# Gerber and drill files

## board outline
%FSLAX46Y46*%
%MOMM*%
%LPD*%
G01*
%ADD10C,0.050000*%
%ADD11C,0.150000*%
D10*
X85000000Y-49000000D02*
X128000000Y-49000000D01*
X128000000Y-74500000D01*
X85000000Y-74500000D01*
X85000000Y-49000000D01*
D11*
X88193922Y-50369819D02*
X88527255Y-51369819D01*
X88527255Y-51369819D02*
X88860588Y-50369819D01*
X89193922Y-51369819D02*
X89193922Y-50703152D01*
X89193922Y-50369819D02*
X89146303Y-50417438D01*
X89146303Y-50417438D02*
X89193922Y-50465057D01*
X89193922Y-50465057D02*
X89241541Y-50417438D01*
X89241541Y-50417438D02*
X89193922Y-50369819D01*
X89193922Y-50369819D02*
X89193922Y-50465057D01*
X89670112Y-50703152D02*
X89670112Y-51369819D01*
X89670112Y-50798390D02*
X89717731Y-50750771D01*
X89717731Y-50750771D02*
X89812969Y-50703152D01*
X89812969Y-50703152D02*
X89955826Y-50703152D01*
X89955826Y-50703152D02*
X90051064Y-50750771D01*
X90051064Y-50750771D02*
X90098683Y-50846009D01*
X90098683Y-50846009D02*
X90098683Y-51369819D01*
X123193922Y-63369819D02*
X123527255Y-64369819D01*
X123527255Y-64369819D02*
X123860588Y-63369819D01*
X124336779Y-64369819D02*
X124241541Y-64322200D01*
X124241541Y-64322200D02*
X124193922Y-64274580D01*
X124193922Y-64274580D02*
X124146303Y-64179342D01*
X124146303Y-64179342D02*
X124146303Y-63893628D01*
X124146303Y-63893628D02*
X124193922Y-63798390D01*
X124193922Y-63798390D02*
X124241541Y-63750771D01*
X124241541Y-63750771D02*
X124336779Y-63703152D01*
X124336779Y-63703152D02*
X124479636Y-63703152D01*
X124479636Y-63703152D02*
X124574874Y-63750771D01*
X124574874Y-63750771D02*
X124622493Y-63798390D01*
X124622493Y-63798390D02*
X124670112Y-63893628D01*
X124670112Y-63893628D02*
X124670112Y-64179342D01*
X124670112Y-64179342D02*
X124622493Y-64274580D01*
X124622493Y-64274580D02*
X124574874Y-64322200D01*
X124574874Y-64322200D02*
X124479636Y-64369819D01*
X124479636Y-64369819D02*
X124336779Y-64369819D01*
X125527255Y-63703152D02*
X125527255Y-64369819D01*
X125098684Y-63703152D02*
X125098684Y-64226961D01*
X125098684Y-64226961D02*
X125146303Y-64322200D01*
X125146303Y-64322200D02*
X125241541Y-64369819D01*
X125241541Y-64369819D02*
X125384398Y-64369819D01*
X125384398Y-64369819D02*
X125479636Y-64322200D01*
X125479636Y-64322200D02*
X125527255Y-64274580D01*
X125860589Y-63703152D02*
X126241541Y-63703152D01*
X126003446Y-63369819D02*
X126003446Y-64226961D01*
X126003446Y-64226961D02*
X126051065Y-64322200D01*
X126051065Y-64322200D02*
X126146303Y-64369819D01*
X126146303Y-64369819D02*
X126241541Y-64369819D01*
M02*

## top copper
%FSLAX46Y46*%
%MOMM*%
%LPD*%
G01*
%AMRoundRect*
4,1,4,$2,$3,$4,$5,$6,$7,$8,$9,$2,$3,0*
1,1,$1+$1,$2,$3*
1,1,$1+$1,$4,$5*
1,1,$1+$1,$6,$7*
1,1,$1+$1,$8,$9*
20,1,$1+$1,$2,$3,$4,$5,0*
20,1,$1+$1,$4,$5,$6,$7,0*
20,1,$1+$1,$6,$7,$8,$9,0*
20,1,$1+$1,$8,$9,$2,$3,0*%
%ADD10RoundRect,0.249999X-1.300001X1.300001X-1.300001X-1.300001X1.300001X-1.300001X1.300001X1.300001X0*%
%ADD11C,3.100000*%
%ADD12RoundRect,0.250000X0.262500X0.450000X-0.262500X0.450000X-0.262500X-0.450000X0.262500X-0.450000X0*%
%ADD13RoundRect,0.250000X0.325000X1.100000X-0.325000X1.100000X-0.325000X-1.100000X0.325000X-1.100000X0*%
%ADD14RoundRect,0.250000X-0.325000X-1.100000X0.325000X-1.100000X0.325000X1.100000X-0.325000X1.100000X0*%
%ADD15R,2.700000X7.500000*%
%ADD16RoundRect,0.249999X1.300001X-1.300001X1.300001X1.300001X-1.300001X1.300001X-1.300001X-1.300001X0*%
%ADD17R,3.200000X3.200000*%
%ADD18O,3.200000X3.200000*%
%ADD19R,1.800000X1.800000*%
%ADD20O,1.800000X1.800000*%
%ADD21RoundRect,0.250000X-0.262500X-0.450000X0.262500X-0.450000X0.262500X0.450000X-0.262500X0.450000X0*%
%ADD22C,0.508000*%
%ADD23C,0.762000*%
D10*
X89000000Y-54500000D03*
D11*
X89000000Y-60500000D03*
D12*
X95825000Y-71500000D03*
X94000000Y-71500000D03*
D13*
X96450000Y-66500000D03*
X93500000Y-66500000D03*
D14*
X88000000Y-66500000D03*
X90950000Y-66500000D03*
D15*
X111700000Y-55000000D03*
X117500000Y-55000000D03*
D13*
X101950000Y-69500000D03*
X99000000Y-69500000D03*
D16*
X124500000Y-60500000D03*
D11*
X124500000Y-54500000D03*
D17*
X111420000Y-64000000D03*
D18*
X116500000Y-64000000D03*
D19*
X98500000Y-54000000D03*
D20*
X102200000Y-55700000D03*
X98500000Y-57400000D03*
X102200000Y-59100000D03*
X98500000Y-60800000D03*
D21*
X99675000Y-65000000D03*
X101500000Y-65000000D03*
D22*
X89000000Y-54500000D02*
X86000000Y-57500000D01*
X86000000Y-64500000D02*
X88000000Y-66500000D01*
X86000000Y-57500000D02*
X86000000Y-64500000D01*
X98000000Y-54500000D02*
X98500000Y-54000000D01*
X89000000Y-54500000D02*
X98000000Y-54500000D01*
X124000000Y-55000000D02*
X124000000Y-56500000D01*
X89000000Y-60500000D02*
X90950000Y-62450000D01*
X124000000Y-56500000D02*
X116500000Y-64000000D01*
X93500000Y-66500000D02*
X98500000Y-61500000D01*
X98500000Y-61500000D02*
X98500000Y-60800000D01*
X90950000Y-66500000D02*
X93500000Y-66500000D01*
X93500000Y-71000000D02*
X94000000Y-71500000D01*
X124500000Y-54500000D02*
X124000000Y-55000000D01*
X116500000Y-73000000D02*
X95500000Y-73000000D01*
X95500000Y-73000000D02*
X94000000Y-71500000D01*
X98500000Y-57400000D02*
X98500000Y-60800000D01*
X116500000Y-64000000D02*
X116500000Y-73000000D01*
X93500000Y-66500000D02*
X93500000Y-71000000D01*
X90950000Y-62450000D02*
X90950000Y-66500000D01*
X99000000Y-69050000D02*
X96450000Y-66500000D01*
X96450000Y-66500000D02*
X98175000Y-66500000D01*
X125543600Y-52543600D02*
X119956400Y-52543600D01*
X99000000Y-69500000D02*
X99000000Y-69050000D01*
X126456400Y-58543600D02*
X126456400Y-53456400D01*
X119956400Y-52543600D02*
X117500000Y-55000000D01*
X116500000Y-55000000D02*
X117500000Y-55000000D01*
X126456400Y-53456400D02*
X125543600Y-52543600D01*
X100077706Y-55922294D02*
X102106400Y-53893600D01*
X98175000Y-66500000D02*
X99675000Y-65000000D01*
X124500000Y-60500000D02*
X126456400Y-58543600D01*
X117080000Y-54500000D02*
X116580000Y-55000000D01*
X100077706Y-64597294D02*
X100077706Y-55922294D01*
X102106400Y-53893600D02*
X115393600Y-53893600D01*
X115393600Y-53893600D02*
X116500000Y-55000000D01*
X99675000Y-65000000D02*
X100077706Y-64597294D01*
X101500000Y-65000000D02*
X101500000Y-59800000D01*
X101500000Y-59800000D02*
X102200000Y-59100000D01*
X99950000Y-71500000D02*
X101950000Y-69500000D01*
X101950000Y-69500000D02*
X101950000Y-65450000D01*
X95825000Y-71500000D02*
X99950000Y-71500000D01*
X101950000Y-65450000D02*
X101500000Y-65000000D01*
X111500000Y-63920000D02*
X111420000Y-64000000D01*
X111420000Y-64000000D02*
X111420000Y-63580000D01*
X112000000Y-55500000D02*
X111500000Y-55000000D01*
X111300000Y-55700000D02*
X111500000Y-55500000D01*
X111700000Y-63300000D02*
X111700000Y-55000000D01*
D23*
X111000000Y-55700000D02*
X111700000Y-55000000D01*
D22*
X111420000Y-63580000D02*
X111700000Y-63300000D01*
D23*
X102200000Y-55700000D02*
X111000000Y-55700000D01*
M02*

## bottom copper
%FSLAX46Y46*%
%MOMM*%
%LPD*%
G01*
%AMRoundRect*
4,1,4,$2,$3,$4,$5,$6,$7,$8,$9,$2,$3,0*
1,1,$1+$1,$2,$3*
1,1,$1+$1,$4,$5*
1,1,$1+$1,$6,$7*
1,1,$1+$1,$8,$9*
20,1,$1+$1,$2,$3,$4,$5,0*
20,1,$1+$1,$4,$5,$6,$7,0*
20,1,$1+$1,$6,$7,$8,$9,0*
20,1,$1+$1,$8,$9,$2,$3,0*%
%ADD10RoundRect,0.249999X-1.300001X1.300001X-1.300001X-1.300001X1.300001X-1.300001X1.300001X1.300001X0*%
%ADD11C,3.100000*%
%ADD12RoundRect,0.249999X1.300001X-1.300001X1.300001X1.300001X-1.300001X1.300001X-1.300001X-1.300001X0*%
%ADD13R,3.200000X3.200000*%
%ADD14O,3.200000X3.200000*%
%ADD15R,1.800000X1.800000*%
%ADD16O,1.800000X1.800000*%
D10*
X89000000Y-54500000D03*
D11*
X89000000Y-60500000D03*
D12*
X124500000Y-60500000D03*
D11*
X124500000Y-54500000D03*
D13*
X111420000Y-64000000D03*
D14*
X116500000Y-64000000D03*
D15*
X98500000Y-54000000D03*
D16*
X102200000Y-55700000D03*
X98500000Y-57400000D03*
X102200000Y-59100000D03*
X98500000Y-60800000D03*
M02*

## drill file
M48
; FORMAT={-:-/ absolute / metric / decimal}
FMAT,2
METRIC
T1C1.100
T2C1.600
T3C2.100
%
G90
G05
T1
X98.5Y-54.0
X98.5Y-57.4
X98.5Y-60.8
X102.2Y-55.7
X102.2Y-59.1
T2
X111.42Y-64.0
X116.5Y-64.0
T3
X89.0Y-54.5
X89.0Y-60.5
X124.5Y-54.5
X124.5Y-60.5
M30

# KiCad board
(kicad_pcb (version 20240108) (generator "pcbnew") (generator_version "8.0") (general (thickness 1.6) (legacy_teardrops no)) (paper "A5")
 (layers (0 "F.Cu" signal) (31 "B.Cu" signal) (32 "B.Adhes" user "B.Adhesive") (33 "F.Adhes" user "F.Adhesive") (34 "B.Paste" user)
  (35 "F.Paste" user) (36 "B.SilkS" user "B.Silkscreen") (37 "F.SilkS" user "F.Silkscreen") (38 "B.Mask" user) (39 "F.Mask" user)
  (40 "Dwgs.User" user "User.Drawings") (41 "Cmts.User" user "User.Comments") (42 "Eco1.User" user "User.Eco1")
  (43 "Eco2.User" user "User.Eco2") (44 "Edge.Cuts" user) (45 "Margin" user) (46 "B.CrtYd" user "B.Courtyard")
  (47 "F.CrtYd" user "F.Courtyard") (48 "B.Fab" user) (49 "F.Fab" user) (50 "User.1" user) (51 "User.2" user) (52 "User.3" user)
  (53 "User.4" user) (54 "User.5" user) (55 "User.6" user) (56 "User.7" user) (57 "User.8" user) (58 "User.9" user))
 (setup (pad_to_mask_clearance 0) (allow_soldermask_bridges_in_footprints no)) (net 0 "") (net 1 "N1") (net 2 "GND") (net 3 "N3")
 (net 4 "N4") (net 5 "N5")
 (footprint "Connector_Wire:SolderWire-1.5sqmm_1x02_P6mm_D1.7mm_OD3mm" (layer "F.Cu") (at 89 54.5 -90)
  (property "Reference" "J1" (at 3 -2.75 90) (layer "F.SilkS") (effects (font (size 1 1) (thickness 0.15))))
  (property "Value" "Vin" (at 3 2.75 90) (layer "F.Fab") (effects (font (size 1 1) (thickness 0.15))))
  (pad "1" thru_hole roundrect (at 0 0 270) (size 3.1 3.1) (drill 2.1) (layers "*.Cu" "*.Mask") (remove_unused_layers no)
   (roundrect_rratio 0.080645) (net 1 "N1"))
  (pad "2" thru_hole circle (at 6 0 270) (size 3.1 3.1) (drill 2.1) (layers "*.Cu" "*.Mask") (remove_unused_layers no) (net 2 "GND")))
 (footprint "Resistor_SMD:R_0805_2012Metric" (layer "F.Cu") (at 94.9125 71.5 180)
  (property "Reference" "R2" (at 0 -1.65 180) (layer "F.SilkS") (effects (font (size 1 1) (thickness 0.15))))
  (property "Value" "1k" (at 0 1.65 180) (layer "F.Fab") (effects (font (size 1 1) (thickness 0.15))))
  (pad "1" smd roundrect (at -0.9125 0 180) (size 1.025 1.4) (layers "F.Cu" "F.Paste" "F.Mask") (roundrect_rratio 0.243902) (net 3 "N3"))
  (pad "2" smd roundrect (at 0.9125 0 180) (size 1.025 1.4) (layers "F.Cu" "F.Paste" "F.Mask") (roundrect_rratio 0.243902) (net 2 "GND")))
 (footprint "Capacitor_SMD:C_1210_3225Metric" (layer "F.Cu") (at 94.975 66.5 180)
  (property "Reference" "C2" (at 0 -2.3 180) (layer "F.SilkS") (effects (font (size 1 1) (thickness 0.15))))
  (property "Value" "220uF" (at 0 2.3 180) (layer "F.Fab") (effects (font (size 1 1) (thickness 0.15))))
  (pad "1" smd roundrect (at -1.475 0 180) (size 1.15 2.7) (layers "F.Cu" "F.Paste" "F.Mask") (roundrect_rratio 0.217391) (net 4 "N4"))
  (pad "2" smd roundrect (at 1.475 0 180) (size 1.15 2.7) (layers "F.Cu" "F.Paste" "F.Mask") (roundrect_rratio 0.217391) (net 2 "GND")))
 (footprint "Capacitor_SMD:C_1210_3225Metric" (layer "F.Cu") (at 89.475 66.5)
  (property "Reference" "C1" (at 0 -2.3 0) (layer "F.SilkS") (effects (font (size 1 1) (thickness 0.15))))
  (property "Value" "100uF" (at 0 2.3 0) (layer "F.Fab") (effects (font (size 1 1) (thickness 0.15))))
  (pad "1" smd roundrect (at -1.475 0) (size 1.15 2.7) (layers "F.Cu" "F.Paste" "F.Mask") (roundrect_rratio 0.217391) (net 1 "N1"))
  (pad "2" smd roundrect (at 1.475 0) (size 1.15 2.7) (layers "F.Cu" "F.Paste" "F.Mask") (roundrect_rratio 0.217391) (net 2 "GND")))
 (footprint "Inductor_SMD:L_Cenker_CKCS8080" (layer "F.Cu") (at 114.6 55)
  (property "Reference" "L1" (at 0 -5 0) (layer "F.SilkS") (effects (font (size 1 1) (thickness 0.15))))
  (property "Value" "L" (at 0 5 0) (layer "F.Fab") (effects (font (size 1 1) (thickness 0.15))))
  (pad "1" smd rect (at -2.9 0) (size 2.7 7.5) (layers "F.Cu" "F.Paste" "F.Mask") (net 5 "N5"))
  (pad "2" smd rect (at 2.9 0) (size 2.7 7.5) (layers "F.Cu" "F.Paste" "F.Mask") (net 4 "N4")))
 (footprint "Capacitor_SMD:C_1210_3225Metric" (layer "F.Cu") (at 100.475 69.5 180)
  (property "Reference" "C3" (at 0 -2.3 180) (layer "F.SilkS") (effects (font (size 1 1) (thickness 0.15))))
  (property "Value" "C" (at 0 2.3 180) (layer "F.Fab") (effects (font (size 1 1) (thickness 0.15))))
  (pad "1" smd roundrect (at -1.475 0 180) (size 1.15 2.7) (layers "F.Cu" "F.Paste" "F.Mask") (roundrect_rratio 0.217391) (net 3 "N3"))
  (pad "2" smd roundrect (at 1.475 0 180) (size 1.15 2.7) (layers "F.Cu" "F.Paste" "F.Mask") (roundrect_rratio 0.217391) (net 4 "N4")))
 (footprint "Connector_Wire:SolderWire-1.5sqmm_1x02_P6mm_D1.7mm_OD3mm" (layer "F.Cu") (at 124.5 60.5 90)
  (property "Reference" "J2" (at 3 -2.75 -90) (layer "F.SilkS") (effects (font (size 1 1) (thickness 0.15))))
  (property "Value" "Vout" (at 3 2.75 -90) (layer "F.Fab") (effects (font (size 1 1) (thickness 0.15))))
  (pad "1" thru_hole roundrect (at 0 0 90) (size 3.1 3.1) (drill 2.1) (layers "*.Cu" "*.Mask") (remove_unused_layers no)
   (roundrect_rratio 0.080645) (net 4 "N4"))
  (pad "2" thru_hole circle (at 6 0 90) (size 3.1 3.1) (drill 2.1) (layers "*.Cu" "*.Mask") (remove_unused_layers no) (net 2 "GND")))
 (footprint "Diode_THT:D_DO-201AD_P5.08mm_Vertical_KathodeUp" (layer "F.Cu") (at 111.42 64)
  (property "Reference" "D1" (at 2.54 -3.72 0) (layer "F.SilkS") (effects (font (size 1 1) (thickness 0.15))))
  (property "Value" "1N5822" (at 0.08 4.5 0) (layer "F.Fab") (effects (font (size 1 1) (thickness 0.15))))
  (pad "1" thru_hole rect (at 0 0) (size 3.2 3.2) (drill 1.6) (layers "*.Cu" "*.Mask") (remove_unused_layers no) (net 5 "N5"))
  (pad "2" thru_hole oval (at 5.08 0) (size 3.2 3.2) (drill 1.6) (layers "*.Cu" "*.Mask") (remove_unused_layers no) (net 2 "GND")))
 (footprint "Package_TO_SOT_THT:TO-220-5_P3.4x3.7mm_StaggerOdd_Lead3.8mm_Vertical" (layer "F.Cu") (at 98.5 54 -90)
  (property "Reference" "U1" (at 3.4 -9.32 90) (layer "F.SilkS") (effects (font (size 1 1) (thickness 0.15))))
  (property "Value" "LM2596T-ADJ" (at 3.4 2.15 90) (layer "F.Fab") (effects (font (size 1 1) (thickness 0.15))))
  (pad "1" thru_hole rect (at 0 0 270) (size 1.8 1.8) (drill 1.1) (layers "*.Cu" "*.Mask") (remove_unused_layers no) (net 1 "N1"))
  (pad "2" thru_hole oval (at 1.7 -3.7 270) (size 1.8 1.8) (drill 1.1) (layers "*.Cu" "*.Mask") (remove_unused_layers no) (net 5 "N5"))
  (pad "3" thru_hole oval (at 3.4 0 270) (size 1.8 1.8) (drill 1.1) (layers "*.Cu" "*.Mask") (remove_unused_layers no) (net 2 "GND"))
  (pad "4" thru_hole oval (at 5.1 -3.7 270) (size 1.8 1.8) (drill 1.1) (layers "*.Cu" "*.Mask") (remove_unused_layers no) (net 3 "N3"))
  (pad "5" thru_hole oval (at 6.8 0 270) (size 1.8 1.8) (drill 1.1) (layers "*.Cu" "*.Mask") (remove_unused_layers no) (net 2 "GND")))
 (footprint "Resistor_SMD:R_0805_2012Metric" (layer "F.Cu") (at 100.5875 65)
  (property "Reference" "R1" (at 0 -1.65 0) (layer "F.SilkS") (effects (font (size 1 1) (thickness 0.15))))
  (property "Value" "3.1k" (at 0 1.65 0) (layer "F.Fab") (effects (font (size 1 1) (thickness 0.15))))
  (pad "1" smd roundrect (at -0.9125 0) (size 1.025 1.4) (layers "F.Cu" "F.Paste" "F.Mask") (roundrect_rratio 0.243902) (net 4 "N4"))
  (pad "2" smd roundrect (at 0.9125 0) (size 1.025 1.4) (layers "F.Cu" "F.Paste" "F.Mask") (roundrect_rratio 0.243902) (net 3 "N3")))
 (gr_rect (start 85 49) (end 128 74.5) (stroke (width 0.05) (type default)) (fill none) (layer "Edge.Cuts"))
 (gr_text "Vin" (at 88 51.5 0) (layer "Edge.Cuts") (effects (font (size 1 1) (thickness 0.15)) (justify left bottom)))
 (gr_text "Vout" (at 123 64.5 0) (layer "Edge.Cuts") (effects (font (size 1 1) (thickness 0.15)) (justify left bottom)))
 (segment (start 89 54.5) (end 86 57.5) (width 0.508) (layer "F.Cu") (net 1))
 (segment (start 86 64.5) (end 88 66.5) (width 0.508) (layer "F.Cu") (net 1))
 (segment (start 86 57.5) (end 86 64.5) (width 0.508) (layer "F.Cu") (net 1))
 (segment (start 98 54.5) (end 98.5 54) (width 0.508) (layer "F.Cu") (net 1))
 (segment (start 89 54.5) (end 98 54.5) (width 0.508) (layer "F.Cu") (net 1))
 (segment (start 124 55) (end 124 56.5) (width 0.508) (layer "F.Cu") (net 2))
 (segment (start 89 60.5) (end 90.95 62.45) (width 0.508) (layer "F.Cu") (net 2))
 (segment (start 124 56.5) (end 116.5 64) (width 0.508) (layer "F.Cu") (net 2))
 (segment (start 93.5 66.5) (end 98.5 61.5) (width 0.508) (layer "F.Cu") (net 2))
 (segment (start 98.5 61.5) (end 98.5 60.8) (width 0.508) (layer "F.Cu") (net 2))
 (segment (start 90.95 66.5) (end 93.5 66.5) (width 0.508) (layer "F.Cu") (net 2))
 (segment (start 93.5 71) (end 94 71.5) (width 0.508) (layer "F.Cu") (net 2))
 (segment (start 124.5 54.5) (end 124 55) (width 0.508) (layer "F.Cu") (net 2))
 (segment (start 116.5 73) (end 95.5 73) (width 0.508) (layer "F.Cu") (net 2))
 (segment (start 95.5 73) (end 94 71.5) (width 0.508) (layer "F.Cu") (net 2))
 (segment (start 98.5 57.4) (end 98.5 60.8) (width 0.508) (layer "F.Cu") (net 2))
 (segment (start 116.5 64) (end 116.5 73) (width 0.508) (layer "F.Cu") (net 2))
 (segment (start 93.5 66.5) (end 93.5 71) (width 0.508) (layer "F.Cu") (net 2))
 (segment (start 90.95 62.45) (end 90.95 66.5) (width 0.508) (layer "F.Cu") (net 2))
 (segment (start 99 69.05) (end 96.45 66.5) (width 0.508) (layer "F.Cu") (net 4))
 (segment (start 96.45 66.5) (end 98.175 66.5) (width 0.508) (layer "F.Cu") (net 4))
 (segment (start 125.5436 52.5436) (end 119.9564 52.5436) (width 0.508) (layer "F.Cu") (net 4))
 (segment (start 99 69.5) (end 99 69.05) (width 0.508) (layer "F.Cu") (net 4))
 (segment (start 126.4564 58.5436) (end 126.4564 53.4564) (width 0.508) (layer "F.Cu") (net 4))
 (segment (start 119.9564 52.5436) (end 117.5 55) (width 0.508) (layer "F.Cu") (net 4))
 (segment (start 116.5 55) (end 117.5 55) (width 0.508) (layer "F.Cu") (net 4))
 (segment (start 126.4564 53.4564) (end 125.5436 52.5436) (width 0.508) (layer "F.Cu") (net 4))
 (segment (start 100.077706 55.922294) (end 102.1064 53.8936) (width 0.508) (layer "F.Cu") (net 4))
 (segment (start 98.175 66.5) (end 99.675 65) (width 0.508) (layer "F.Cu") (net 4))
 (segment (start 124.5 60.5) (end 126.4564 58.5436) (width 0.508) (layer "F.Cu") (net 4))
 (segment (start 117.08 54.5) (end 116.58 55) (width 0.508) (layer "F.Cu") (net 4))
 (segment (start 100.077706 64.597294) (end 100.077706 55.922294) (width 0.508) (layer "F.Cu") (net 4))
 (segment (start 102.1064 53.8936) (end 115.3936 53.8936) (width 0.508) (layer "F.Cu") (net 4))
 (segment (start 115.3936 53.8936) (end 116.5 55) (width 0.508) (layer "F.Cu") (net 4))
 (segment (start 99.675 65) (end 100.077706 64.597294) (width 0.508) (layer "F.Cu") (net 4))
 (segment (start 101.5 65) (end 101.5 59.8) (width 0.508) (layer "F.Cu") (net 3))
 (segment (start 101.5 59.8) (end 102.2 59.1) (width 0.508) (layer "F.Cu") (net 3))
 (segment (start 99.95 71.5) (end 101.95 69.5) (width 0.508) (layer "F.Cu") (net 3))
 (segment (start 101.95 69.5) (end 101.95 65.45) (width 0.508) (layer "F.Cu") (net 3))
 (segment (start 95.825 71.5) (end 99.95 71.5) (width 0.508) (layer "F.Cu") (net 3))
 (segment (start 101.95 65.45) (end 101.5 65) (width 0.508) (layer "F.Cu") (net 3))
 (segment (start 111.5 63.92) (end 111.42 64) (width 0.508) (layer "F.Cu") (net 5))
 (segment (start 111.42 64) (end 111.42 63.58) (width 0.508) (layer "F.Cu") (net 5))
 (segment (start 112 55.5) (end 111.5 55) (width 0.508) (layer "F.Cu") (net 5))
 (segment (start 111.3 55.7) (end 111.5 55.5) (width 0.508) (layer "F.Cu") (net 5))
 (segment (start 111.7 63.3) (end 111.7 55) (width 0.508) (layer "F.Cu") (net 5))
 (segment (start 111 55.7) (end 111.7 55) (width 0.762) (layer "F.Cu") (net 5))
 (segment (start 111.42 63.58) (end 111.7 63.3) (width 0.508) (layer "F.Cu") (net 5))
 (segment (start 102.2 55.7) (end 111 55.7) (width 0.762) (layer "F.Cu") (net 5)))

